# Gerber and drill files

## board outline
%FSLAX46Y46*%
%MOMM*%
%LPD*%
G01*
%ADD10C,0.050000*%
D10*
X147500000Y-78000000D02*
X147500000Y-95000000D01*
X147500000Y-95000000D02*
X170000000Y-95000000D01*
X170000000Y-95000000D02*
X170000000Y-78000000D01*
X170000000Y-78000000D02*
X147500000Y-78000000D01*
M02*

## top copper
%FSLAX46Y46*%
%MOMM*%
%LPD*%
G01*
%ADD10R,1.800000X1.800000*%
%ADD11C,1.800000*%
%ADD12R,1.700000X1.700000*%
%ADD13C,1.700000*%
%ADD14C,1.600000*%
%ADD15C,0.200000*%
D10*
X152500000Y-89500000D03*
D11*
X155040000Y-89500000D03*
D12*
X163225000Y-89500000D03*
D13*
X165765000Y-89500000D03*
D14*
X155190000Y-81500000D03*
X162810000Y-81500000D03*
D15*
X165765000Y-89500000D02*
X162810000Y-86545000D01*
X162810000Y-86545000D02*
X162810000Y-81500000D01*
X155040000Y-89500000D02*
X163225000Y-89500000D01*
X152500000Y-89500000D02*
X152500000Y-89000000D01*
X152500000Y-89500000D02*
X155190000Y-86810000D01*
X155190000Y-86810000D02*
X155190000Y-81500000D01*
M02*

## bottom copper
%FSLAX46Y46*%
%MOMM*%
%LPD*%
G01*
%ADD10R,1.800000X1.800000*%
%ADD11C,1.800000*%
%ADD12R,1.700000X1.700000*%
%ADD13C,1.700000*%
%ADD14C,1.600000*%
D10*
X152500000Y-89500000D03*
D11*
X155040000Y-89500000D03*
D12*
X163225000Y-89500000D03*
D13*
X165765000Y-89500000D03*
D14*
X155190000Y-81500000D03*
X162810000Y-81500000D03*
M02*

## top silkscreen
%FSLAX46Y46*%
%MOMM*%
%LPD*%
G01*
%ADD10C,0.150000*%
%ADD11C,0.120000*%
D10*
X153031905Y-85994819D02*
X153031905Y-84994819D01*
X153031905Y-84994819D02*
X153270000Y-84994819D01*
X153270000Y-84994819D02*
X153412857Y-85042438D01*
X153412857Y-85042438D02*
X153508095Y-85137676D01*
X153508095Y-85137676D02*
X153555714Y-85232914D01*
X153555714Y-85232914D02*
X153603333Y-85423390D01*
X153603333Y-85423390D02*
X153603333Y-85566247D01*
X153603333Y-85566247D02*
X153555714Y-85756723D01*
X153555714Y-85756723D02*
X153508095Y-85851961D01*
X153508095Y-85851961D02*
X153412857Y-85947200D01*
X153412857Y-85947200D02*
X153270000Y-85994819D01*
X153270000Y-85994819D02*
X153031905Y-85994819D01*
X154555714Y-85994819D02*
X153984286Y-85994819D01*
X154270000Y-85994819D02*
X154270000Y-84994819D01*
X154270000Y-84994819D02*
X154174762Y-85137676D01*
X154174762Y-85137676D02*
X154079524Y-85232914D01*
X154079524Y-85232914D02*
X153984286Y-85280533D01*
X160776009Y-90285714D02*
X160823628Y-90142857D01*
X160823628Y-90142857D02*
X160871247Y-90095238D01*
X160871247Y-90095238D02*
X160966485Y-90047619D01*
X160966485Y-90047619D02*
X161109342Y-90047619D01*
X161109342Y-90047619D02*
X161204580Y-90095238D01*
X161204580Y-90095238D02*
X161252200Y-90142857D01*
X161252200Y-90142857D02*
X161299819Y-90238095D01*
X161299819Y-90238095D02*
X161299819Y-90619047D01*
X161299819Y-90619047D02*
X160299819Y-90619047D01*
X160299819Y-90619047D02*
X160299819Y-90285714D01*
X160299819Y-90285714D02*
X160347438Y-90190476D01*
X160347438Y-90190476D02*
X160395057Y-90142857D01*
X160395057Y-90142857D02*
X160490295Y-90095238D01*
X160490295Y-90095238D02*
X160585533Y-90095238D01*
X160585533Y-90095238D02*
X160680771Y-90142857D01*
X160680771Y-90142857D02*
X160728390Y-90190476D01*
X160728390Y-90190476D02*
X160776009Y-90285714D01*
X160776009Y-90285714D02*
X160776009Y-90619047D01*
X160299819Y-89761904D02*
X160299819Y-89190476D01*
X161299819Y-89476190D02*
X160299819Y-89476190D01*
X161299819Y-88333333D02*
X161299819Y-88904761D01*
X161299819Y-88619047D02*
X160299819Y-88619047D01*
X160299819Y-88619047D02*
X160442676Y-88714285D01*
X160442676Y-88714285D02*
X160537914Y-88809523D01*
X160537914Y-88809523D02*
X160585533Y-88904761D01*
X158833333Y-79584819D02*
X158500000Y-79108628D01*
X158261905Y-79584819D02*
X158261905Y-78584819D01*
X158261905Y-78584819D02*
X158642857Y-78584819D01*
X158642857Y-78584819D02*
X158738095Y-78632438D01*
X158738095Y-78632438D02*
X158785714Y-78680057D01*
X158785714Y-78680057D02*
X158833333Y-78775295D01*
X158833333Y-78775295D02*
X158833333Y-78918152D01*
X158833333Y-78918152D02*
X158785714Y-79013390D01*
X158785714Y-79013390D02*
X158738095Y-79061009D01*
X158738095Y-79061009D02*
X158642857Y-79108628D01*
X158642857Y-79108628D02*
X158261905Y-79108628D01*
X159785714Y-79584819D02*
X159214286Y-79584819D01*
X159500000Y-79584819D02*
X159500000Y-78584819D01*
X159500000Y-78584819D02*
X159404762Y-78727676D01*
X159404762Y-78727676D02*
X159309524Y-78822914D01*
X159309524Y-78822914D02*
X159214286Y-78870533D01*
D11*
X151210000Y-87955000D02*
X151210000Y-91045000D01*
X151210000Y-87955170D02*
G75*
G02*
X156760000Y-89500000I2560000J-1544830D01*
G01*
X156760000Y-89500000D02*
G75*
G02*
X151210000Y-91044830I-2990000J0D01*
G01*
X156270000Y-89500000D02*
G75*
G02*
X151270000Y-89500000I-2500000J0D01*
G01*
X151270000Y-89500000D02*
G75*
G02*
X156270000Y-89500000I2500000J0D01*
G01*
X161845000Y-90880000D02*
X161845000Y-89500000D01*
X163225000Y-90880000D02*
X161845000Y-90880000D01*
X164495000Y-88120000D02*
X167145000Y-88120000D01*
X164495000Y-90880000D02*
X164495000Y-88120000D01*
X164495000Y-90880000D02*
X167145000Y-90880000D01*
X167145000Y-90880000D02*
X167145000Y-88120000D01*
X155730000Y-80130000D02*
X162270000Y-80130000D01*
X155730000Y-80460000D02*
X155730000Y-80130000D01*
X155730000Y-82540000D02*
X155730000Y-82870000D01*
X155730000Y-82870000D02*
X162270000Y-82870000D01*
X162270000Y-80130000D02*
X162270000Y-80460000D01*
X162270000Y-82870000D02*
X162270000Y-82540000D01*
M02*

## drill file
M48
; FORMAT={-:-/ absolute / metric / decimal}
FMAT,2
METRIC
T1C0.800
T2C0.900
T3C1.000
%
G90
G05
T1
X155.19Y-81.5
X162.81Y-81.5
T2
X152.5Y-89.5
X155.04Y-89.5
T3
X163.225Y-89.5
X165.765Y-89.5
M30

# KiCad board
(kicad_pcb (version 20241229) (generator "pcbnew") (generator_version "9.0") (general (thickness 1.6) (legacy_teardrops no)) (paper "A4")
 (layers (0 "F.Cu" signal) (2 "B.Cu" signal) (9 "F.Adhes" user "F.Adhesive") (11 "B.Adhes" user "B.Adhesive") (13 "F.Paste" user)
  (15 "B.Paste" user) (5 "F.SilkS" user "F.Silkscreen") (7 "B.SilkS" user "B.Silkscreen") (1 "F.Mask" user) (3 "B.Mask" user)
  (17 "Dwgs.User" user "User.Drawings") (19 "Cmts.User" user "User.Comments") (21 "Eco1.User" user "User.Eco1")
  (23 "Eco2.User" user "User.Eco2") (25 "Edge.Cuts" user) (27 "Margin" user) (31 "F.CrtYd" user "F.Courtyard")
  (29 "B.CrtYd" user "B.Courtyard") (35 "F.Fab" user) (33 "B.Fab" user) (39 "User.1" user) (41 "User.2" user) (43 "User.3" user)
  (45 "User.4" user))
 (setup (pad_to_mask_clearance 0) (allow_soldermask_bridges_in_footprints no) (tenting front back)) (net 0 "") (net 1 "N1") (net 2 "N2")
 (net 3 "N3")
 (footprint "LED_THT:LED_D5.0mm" (layer "F.Cu") (at 152.5 89.5)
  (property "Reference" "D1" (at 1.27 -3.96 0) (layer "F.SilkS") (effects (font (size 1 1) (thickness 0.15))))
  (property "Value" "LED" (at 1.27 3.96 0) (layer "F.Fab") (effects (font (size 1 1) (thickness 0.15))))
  (fp_line (start -1.29 -1.545) (end -1.29 1.545) (stroke (width 0.12) (type solid)) (layer "F.SilkS"))
  (fp_arc (start -1.29 -1.54483) (mid 2.071779 -2.880495) (end 4.26 0) (stroke (width 0.12) (type solid)) (layer "F.SilkS"))
  (fp_arc (start 4.26 0) (mid 2.071779 2.880495) (end -1.29 1.54483) (stroke (width 0.12) (type solid)) (layer "F.SilkS"))
  (fp_circle (center 1.27 0) (end 3.77 0) (stroke (width 0.12) (type solid)) (fill no) (layer "F.SilkS"))
  (pad "1" thru_hole rect (at 0 0) (size 1.8 1.8) (drill 0.9) (layers "*.Cu" "*.Mask") (remove_unused_layers no) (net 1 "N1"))
  (pad "2" thru_hole circle (at 2.54 0) (size 1.8 1.8) (drill 0.9) (layers "*.Cu" "*.Mask") (remove_unused_layers no) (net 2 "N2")))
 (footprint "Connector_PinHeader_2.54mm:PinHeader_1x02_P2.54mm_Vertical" (layer "F.Cu") (at 163.225 89.5 90)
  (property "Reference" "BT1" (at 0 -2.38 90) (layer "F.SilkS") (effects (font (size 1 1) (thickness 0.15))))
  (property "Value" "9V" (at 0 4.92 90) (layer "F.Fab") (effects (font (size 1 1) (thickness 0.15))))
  (fp_line (start -1.38 -1.38) (end 0 -1.38) (stroke (width 0.12) (type solid)) (layer "F.SilkS"))
  (fp_line (start -1.38 0) (end -1.38 -1.38) (stroke (width 0.12) (type solid)) (layer "F.SilkS"))
  (fp_line (start 1.38 1.27) (end 1.38 3.92) (stroke (width 0.12) (type solid)) (layer "F.SilkS"))
  (fp_line (start -1.38 1.27) (end 1.38 1.27) (stroke (width 0.12) (type solid)) (layer "F.SilkS"))
  (fp_line (start -1.38 1.27) (end -1.38 3.92) (stroke (width 0.12) (type solid)) (layer "F.SilkS"))
  (fp_line (start -1.38 3.92) (end 1.38 3.92) (stroke (width 0.12) (type solid)) (layer "F.SilkS"))
  (pad "1" thru_hole rect (at 0 0 90) (size 1.7 1.7) (drill 1) (layers "*.Cu" "*.Mask") (remove_unused_layers no) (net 2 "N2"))
  (pad "2" thru_hole circle (at 0 2.54 90) (size 1.7 1.7) (drill 1) (layers "*.Cu" "*.Mask") (remove_unused_layers no) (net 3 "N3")))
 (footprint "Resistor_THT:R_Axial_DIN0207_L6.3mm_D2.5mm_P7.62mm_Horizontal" (layer "F.Cu") (at 155.19 81.5)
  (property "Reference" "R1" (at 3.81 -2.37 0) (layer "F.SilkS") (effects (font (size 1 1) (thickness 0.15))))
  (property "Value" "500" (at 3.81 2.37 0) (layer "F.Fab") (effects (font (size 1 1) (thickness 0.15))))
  (fp_line (start 0.54 -1.37) (end 7.08 -1.37) (stroke (width 0.12) (type solid)) (layer "F.SilkS"))
  (fp_line (start 0.54 -1.04) (end 0.54 -1.37) (stroke (width 0.12) (type solid)) (layer "F.SilkS"))
  (fp_line (start 0.54 1.04) (end 0.54 1.37) (stroke (width 0.12) (type solid)) (layer "F.SilkS"))
  (fp_line (start 0.54 1.37) (end 7.08 1.37) (stroke (width 0.12) (type solid)) (layer "F.SilkS"))
  (fp_line (start 7.08 -1.37) (end 7.08 -1.04) (stroke (width 0.12) (type solid)) (layer "F.SilkS"))
  (fp_line (start 7.08 1.37) (end 7.08 1.04) (stroke (width 0.12) (type solid)) (layer "F.SilkS"))
  (pad "1" thru_hole circle (at 0 0) (size 1.6 1.6) (drill 0.8) (layers "*.Cu" "*.Mask") (remove_unused_layers no) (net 1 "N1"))
  (pad "2" thru_hole circle (at 7.62 0) (size 1.6 1.6) (drill 0.8) (layers "*.Cu" "*.Mask") (remove_unused_layers no) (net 3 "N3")))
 (gr_line (start 147.5 78) (end 147.5 95) (stroke (width 0.05) (type default)) (layer "Edge.Cuts"))
 (gr_line (start 147.5 95) (end 170 95) (stroke (width 0.05) (type default)) (layer "Edge.Cuts"))
 (gr_line (start 170 95) (end 170 78) (stroke (width 0.05) (type default)) (layer "Edge.Cuts"))
 (gr_line (start 170 78) (end 147.5 78) (stroke (width 0.05) (type default)) (layer "Edge.Cuts"))
 (segment (start 165.765 89.5) (end 162.81 86.545) (width 0.2) (layer "F.Cu") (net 3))
 (segment (start 162.81 86.545) (end 162.81 81.5) (width 0.2) (layer "F.Cu") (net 3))
 (segment (start 155.04 89.5) (end 163.225 89.5) (width 0.2) (layer "F.Cu") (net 2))
 (segment (start 152.5 89.5) (end 152.5 89) (width 0.2) (layer "F.Cu") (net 1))
 (segment (start 152.5 89.5) (end 155.19 86.81) (width 0.2) (layer "F.Cu") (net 1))
 (segment (start 155.19 86.81) (end 155.19 81.5) (width 0.2) (layer "F.Cu") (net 1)))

